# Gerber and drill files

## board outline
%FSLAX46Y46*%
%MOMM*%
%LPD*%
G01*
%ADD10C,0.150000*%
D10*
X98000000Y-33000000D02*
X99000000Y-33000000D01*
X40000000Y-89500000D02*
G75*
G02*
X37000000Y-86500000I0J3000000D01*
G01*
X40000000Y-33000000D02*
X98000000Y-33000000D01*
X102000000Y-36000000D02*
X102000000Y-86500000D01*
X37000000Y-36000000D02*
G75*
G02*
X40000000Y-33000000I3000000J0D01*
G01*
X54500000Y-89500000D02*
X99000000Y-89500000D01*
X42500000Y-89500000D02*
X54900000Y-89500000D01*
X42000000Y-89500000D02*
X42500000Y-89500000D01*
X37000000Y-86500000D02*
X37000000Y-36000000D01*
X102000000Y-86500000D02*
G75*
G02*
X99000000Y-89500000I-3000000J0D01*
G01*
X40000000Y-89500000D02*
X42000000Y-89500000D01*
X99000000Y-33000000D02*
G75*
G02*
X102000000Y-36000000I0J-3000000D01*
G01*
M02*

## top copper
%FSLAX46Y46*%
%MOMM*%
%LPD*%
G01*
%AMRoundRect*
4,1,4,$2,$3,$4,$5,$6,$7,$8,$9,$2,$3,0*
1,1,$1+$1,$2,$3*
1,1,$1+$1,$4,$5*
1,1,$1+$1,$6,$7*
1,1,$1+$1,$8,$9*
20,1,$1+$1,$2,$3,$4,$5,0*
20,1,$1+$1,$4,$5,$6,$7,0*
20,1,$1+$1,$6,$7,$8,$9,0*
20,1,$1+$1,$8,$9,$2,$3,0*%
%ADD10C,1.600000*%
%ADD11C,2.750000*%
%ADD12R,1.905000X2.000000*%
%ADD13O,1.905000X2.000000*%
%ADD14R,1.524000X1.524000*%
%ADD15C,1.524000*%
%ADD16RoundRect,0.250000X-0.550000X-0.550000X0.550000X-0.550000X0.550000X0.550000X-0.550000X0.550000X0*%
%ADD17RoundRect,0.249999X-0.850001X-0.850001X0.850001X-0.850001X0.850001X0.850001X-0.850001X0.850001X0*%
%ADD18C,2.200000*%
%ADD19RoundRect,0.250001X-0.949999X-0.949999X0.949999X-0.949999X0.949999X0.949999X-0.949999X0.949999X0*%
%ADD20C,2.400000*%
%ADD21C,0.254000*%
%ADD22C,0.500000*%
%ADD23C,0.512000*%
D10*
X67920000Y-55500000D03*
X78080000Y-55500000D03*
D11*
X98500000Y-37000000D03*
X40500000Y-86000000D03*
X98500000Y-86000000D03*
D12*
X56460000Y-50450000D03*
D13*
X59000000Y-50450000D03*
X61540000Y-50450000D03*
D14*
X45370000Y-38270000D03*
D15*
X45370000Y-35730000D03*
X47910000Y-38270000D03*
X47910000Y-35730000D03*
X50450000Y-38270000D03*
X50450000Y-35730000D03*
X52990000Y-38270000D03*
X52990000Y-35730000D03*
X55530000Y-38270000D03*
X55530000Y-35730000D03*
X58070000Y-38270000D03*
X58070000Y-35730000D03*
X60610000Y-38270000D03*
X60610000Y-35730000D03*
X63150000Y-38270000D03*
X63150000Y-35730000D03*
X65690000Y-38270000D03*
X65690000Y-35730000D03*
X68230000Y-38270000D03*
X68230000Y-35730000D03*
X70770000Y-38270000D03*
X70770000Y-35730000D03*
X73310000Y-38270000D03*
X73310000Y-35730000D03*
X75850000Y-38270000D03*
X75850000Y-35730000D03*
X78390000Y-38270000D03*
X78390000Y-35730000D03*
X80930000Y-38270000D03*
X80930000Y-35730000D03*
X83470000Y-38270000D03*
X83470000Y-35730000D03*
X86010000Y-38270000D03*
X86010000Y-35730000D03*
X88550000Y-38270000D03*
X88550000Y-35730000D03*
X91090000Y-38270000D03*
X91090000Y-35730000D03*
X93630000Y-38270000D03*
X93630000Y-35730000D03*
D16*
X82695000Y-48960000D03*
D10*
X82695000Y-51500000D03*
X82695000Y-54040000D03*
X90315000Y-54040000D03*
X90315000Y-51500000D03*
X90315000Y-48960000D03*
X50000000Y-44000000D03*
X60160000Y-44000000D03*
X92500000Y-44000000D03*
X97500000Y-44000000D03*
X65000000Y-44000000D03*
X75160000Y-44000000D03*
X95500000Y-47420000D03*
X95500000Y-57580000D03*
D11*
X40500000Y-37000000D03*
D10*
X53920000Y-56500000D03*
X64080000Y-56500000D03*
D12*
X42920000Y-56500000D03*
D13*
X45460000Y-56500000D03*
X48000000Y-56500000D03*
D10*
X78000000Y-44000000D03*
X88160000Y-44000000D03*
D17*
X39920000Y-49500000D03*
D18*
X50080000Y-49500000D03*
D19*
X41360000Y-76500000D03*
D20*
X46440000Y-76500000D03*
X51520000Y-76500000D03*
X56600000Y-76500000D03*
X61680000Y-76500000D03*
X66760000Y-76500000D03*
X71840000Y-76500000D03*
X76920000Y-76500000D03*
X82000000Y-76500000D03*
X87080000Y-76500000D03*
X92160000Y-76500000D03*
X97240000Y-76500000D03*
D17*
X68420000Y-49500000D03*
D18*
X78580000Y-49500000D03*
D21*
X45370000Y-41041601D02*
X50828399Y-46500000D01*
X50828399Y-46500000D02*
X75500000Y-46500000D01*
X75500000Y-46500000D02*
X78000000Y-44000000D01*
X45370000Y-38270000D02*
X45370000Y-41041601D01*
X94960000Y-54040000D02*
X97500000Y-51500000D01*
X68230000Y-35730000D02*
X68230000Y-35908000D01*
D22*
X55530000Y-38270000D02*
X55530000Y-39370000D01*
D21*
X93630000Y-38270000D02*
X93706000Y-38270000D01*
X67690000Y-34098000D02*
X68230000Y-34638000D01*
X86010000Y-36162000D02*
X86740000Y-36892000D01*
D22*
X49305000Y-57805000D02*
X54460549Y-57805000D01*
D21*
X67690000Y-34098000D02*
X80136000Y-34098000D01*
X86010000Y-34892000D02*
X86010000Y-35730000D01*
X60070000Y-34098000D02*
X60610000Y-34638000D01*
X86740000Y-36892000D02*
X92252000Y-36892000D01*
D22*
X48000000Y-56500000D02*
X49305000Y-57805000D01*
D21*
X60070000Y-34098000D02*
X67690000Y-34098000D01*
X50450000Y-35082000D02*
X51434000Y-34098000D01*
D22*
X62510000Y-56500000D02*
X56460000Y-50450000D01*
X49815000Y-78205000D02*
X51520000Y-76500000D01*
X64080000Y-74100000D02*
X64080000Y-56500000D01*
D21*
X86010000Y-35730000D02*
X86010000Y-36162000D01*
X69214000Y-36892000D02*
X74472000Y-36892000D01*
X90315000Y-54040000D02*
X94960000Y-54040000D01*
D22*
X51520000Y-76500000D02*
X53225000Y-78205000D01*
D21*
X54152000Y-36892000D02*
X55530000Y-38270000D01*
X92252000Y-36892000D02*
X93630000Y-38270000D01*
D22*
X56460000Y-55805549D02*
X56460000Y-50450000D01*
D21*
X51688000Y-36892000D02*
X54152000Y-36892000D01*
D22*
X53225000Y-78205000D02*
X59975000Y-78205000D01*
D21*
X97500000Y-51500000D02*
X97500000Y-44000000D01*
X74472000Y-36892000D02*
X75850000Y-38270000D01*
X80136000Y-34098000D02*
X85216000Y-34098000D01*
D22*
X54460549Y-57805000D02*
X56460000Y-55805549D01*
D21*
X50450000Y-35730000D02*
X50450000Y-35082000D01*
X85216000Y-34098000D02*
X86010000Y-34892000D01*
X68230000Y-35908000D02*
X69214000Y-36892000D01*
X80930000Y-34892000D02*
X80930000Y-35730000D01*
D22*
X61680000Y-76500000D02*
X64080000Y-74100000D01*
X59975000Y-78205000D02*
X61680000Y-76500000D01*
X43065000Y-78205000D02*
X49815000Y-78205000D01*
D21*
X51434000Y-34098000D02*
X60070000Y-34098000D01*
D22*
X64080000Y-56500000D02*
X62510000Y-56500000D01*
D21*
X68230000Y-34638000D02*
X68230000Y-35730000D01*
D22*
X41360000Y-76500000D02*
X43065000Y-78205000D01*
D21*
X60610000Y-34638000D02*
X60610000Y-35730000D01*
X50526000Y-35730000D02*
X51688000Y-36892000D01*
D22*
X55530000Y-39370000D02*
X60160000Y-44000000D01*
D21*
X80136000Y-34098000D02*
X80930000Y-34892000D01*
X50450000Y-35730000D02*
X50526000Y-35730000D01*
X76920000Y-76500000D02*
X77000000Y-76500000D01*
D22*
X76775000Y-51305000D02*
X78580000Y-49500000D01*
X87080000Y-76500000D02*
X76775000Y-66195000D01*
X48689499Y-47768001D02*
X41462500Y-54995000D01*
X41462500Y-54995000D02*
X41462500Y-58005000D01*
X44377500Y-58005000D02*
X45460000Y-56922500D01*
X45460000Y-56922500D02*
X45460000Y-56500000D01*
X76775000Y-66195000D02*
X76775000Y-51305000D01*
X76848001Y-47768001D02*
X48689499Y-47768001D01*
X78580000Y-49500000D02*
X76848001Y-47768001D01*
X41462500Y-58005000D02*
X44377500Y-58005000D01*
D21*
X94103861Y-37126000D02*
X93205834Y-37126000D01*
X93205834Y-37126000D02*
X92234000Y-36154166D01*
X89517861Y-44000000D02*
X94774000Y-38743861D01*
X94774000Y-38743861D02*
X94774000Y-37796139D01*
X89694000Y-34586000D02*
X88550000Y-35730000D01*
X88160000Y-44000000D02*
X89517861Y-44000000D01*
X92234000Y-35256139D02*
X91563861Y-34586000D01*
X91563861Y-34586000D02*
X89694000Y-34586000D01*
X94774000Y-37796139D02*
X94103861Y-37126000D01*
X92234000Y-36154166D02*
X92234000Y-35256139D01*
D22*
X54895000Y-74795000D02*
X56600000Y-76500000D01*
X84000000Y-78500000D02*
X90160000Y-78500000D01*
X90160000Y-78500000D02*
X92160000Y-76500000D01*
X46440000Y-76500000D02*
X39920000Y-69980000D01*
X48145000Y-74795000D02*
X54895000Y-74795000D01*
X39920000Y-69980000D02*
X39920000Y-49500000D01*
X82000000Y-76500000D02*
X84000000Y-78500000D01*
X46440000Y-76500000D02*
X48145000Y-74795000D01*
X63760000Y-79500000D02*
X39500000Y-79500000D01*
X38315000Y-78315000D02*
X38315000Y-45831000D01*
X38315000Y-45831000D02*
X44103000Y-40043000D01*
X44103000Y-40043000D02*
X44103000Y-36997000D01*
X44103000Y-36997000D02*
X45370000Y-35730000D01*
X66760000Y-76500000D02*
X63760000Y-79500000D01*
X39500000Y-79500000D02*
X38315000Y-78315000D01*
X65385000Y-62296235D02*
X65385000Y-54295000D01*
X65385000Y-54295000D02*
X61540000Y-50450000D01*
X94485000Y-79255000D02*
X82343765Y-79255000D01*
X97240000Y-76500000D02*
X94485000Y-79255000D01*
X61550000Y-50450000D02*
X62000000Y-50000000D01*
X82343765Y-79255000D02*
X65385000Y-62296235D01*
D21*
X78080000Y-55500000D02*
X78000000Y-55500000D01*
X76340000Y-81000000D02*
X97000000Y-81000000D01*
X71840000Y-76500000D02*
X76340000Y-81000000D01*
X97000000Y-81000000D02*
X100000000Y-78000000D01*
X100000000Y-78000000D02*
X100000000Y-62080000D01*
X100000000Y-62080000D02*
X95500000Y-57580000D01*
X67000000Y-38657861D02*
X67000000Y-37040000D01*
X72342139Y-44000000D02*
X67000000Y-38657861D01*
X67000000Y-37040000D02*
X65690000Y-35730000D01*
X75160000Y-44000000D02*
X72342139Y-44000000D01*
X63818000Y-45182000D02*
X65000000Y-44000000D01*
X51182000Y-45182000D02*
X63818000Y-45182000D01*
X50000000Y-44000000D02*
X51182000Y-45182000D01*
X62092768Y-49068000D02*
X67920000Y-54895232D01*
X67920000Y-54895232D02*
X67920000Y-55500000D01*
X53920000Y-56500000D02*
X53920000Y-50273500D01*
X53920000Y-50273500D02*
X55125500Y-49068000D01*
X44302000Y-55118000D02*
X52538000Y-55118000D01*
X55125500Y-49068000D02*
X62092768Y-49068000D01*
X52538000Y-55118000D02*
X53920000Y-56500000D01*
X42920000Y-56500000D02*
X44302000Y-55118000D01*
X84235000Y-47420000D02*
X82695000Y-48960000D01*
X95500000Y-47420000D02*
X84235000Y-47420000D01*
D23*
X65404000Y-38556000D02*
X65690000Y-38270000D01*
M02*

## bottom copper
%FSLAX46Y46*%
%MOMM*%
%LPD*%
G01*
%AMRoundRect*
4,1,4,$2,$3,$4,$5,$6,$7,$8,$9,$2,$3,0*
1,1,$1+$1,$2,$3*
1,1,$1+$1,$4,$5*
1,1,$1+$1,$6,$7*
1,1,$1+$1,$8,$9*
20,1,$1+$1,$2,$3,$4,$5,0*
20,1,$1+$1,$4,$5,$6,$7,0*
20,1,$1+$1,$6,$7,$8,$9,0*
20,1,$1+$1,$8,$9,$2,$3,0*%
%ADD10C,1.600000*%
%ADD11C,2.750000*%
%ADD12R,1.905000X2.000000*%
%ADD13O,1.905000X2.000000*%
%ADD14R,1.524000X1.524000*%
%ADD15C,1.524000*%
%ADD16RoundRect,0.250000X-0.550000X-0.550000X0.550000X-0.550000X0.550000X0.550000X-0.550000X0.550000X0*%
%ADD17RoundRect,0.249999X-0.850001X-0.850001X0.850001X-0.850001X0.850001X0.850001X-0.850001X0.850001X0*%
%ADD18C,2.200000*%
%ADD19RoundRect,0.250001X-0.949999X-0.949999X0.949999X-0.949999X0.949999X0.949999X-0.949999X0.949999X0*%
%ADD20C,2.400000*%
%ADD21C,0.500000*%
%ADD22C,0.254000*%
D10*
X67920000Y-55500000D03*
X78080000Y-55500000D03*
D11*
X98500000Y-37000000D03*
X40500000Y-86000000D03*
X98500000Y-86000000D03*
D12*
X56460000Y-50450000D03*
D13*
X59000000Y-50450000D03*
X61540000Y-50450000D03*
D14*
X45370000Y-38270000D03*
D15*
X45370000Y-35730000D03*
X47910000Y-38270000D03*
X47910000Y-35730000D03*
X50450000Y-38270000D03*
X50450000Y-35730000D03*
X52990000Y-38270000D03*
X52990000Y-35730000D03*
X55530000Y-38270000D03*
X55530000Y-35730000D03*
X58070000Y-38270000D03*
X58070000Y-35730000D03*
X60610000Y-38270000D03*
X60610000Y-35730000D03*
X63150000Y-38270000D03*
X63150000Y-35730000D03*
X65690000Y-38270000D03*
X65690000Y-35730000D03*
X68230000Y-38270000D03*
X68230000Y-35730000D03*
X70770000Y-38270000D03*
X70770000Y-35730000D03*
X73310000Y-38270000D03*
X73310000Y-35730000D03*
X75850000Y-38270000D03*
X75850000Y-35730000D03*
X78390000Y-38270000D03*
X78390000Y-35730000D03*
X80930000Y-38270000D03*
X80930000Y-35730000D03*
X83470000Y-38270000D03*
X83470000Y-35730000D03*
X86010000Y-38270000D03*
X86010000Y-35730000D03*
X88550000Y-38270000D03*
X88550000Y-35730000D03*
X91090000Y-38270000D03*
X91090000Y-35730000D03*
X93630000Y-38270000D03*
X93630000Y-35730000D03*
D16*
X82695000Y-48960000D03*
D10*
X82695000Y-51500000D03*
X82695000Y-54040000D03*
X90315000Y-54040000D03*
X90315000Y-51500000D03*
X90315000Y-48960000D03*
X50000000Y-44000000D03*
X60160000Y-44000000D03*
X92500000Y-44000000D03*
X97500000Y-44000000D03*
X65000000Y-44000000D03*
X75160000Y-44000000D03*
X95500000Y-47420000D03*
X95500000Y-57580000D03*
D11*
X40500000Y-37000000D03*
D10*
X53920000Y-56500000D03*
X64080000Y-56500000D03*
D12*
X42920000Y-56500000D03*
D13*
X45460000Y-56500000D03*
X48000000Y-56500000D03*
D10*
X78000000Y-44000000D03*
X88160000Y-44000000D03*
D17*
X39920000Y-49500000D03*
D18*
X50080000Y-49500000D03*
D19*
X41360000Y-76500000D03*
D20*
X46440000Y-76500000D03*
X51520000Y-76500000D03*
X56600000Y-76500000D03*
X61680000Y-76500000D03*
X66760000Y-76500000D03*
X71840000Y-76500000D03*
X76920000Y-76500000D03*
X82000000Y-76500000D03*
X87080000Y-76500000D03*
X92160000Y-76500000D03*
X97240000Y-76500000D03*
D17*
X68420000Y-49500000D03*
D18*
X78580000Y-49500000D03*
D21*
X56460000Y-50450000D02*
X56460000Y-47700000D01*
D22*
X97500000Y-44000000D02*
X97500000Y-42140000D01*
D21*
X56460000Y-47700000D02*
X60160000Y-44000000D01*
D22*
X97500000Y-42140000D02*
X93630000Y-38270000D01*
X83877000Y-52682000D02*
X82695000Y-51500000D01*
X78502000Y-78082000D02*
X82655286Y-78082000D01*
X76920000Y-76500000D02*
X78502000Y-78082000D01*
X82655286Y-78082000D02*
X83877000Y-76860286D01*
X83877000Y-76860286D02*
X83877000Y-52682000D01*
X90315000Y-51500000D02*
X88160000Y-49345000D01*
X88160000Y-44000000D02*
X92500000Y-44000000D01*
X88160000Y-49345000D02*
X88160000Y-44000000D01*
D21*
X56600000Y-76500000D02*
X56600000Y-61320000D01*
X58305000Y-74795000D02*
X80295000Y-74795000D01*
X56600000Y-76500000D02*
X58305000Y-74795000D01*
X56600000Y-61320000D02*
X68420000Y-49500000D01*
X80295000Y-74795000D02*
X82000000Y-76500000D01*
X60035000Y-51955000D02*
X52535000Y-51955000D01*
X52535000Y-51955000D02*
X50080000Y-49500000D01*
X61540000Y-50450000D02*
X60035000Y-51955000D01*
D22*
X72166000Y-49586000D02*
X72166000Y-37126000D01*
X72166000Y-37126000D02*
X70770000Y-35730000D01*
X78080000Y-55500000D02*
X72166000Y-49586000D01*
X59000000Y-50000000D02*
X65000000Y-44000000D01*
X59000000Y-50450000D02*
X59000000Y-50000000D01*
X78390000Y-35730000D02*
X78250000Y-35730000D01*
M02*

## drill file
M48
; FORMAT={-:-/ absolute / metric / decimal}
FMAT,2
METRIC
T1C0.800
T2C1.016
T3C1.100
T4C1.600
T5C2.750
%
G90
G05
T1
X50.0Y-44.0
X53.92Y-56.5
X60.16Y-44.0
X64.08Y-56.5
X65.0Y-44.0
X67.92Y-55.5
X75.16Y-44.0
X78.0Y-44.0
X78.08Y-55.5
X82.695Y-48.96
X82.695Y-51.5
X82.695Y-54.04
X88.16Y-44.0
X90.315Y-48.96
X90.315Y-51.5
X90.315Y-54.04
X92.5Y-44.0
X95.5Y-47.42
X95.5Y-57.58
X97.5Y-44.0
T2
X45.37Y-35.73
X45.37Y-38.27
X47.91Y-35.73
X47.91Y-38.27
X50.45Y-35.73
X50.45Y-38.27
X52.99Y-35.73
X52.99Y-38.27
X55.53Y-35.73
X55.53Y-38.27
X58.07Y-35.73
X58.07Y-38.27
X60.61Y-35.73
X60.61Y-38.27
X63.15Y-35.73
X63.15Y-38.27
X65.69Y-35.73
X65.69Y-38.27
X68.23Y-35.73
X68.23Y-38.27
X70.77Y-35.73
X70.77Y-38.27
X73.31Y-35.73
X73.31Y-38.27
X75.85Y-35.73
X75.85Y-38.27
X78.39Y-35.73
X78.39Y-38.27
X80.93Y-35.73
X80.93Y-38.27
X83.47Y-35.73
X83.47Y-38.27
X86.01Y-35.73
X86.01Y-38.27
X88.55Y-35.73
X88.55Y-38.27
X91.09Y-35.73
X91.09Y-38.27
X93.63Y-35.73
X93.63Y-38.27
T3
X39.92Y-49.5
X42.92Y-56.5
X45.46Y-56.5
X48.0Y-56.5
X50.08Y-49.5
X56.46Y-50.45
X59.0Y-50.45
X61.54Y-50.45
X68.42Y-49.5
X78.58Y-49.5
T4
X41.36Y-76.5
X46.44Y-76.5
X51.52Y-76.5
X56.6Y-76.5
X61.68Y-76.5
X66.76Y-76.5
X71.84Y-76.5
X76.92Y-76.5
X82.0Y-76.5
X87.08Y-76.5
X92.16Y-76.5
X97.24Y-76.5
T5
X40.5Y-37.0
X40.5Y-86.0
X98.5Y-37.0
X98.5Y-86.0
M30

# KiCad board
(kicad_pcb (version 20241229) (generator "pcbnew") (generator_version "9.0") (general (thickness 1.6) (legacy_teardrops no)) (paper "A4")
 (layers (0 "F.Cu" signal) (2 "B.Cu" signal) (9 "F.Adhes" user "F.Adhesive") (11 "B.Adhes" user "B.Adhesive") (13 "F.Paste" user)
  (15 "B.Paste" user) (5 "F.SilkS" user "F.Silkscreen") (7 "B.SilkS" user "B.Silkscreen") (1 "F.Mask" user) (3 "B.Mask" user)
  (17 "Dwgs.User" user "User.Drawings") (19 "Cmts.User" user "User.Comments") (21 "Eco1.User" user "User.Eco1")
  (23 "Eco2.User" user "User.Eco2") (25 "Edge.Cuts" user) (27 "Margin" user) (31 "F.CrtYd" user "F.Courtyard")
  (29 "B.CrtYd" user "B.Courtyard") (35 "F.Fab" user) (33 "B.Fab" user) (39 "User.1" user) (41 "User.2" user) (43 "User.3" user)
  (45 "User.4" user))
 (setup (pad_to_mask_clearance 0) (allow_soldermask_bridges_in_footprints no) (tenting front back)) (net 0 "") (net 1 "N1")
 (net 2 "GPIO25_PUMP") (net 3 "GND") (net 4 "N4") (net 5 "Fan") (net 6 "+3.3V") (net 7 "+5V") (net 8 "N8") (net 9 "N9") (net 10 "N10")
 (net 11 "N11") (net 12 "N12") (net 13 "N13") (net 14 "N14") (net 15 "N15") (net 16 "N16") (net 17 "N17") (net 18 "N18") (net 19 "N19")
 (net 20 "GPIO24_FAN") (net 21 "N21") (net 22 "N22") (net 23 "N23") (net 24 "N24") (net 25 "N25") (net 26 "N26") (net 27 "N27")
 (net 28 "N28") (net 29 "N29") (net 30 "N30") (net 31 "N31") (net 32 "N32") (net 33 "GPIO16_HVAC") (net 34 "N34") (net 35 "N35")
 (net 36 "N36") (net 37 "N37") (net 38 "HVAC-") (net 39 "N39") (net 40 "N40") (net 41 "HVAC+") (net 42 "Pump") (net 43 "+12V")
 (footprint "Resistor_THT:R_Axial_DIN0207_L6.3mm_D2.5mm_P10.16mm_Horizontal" (layer "F.Cu") (at 67.92 55.5)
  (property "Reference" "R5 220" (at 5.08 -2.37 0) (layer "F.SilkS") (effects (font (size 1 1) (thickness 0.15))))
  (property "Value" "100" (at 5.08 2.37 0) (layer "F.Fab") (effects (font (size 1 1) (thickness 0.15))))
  (pad "1" thru_hole circle (at 0 0) (size 1.6 1.6) (drill 0.8) (layers "*.Cu" "*.Mask") (remove_unused_layers no) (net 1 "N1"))
  (pad "2" thru_hole circle (at 10.16 0) (size 1.6 1.6) (drill 0.8) (layers "*.Cu" "*.Mask") (remove_unused_layers no) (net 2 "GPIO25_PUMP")))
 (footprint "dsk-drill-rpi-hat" (layer "F.Cu") (at 98.5 37)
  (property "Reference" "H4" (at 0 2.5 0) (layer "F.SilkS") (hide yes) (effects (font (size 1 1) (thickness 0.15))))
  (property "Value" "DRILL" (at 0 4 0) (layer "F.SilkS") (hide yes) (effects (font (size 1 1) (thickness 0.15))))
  (pad "1" thru_hole circle (at 0 0) (size 2.75 2.75) (drill 2.75) (layers "*.Cu") (remove_unused_layers no) (solder_mask_margin 1.725)
   (clearance 1.725) (zone_connect 0)))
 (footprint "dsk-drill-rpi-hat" (layer "F.Cu") (at 40.5 86)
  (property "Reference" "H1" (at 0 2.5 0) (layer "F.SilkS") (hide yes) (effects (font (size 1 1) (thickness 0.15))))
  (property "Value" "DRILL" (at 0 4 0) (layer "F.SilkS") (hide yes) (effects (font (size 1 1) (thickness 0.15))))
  (pad "1" thru_hole circle (at 0 0) (size 2.75 2.75) (drill 2.75) (layers "*.Cu") (remove_unused_layers no) (solder_mask_margin 1.725)
   (clearance 1.725) (zone_connect 0)))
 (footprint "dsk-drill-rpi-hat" (layer "F.Cu") (at 98.5 86)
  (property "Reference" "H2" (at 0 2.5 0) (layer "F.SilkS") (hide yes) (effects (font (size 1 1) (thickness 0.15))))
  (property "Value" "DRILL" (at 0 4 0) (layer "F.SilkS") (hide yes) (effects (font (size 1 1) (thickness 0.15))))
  (pad "1" thru_hole circle (at 0 0) (size 2.75 2.75) (drill 2.75) (layers "*.Cu") (remove_unused_layers no) (solder_mask_margin 1.725)
   (clearance 1.725) (zone_connect 0)))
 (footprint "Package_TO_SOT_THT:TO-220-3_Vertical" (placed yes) (layer "F.Cu") (at 56.46 50.45)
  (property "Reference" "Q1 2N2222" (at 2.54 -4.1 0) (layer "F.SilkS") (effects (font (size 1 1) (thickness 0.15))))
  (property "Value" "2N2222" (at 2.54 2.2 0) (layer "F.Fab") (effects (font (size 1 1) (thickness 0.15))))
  (pad "1" thru_hole rect (at 0 0) (size 1.905 2) (drill 1.1) (layers "*.Cu" "*.Mask") (remove_unused_layers no) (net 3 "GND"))
  (pad "2" thru_hole oval (at 2.54 0) (size 1.905 2) (drill 1.1) (layers "*.Cu" "*.Mask") (remove_unused_layers no) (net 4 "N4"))
  (pad "3" thru_hole oval (at 5.08 0) (size 1.905 2) (drill 1.1) (layers "*.Cu" "*.Mask") (remove_unused_layers no) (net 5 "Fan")))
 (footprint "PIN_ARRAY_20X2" (layer "F.Cu") (at 69.5 37)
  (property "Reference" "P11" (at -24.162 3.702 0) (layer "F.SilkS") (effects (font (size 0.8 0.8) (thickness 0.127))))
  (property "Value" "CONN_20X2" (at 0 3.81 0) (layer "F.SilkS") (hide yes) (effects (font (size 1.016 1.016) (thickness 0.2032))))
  (pad "1" thru_hole rect (at -24.13 1.27) (size 1.524 1.524) (drill 1.016) (layers "*.Cu" "*.Mask" "F.SilkS") (remove_unused_layers no)
   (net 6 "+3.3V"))
  (pad "2" thru_hole circle (at -24.13 -1.27) (size 1.524 1.524) (drill 1.016) (layers "*.Cu" "*.Mask" "F.SilkS") (remove_unused_layers no)
   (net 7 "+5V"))
  (pad "3" thru_hole circle (at -21.59 1.27) (size 1.524 1.524) (drill 1.016) (layers "*.Cu" "*.Mask" "F.SilkS") (remove_unused_layers no)
   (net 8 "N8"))
  (pad "4" thru_hole circle (at -21.59 -1.27) (size 1.524 1.524) (drill 1.016) (layers "*.Cu" "*.Mask" "F.SilkS") (remove_unused_layers no)
   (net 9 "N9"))
  (pad "5" thru_hole circle (at -19.05 1.27) (size 1.524 1.524) (drill 1.016) (layers "*.Cu" "*.Mask" "F.SilkS") (remove_unused_layers no)
   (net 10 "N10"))
  (pad "6" thru_hole circle (at -19.05 -1.27) (size 1.524 1.524) (drill 1.016) (layers "*.Cu" "*.Mask" "F.SilkS") (remove_unused_layers no)
   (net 3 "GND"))
  (pad "7" thru_hole circle (at -16.51 1.27) (size 1.524 1.524) (drill 1.016) (layers "*.Cu" "*.Mask" "F.SilkS") (remove_unused_layers no)
   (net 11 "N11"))
  (pad "8" thru_hole circle (at -16.51 -1.27) (size 1.524 1.524) (drill 1.016) (layers "*.Cu" "*.Mask" "F.SilkS") (remove_unused_layers no)
   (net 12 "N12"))
  (pad "9" thru_hole circle (at -13.97 1.27) (size 1.524 1.524) (drill 1.016) (layers "*.Cu" "*.Mask" "F.SilkS") (remove_unused_layers no)
   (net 3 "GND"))
  (pad "10" thru_hole circle (at -13.97 -1.27) (size 1.524 1.524) (drill 1.016) (layers "*.Cu" "*.Mask" "F.SilkS") (remove_unused_layers no)
   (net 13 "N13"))
  (pad "11" thru_hole circle (at -11.43 1.27) (size 1.524 1.524) (drill 1.016) (layers "*.Cu" "*.Mask" "F.SilkS") (remove_unused_layers no)
   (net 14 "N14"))
  (pad "12" thru_hole circle (at -11.43 -1.27) (size 1.524 1.524) (drill 1.016) (layers "*.Cu" "*.Mask" "F.SilkS") (remove_unused_layers no)
   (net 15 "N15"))
  (pad "13" thru_hole circle (at -8.89 1.27) (size 1.524 1.524) (drill 1.016) (layers "*.Cu" "*.Mask" "F.SilkS") (remove_unused_layers no)
   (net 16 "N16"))
  (pad "14" thru_hole circle (at -8.89 -1.27) (size 1.524 1.524) (drill 1.016) (layers "*.Cu" "*.Mask" "F.SilkS") (remove_unused_layers no)
   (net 3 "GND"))
  (pad "15" thru_hole circle (at -6.35 1.27) (size 1.524 1.524) (drill 1.016) (layers "*.Cu" "*.Mask" "F.SilkS") (remove_unused_layers no)
   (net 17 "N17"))
  (pad "16" thru_hole circle (at -6.35 -1.27) (size 1.524 1.524) (drill 1.016) (layers "*.Cu" "*.Mask" "F.SilkS") (remove_unused_layers no)
   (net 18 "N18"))
  (pad "17" thru_hole circle (at -3.81 1.27) (size 1.524 1.524) (drill 1.016) (layers "*.Cu" "*.Mask" "F.SilkS") (remove_unused_layers no)
   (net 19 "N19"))
  (pad "18" thru_hole circle (at -3.81 -1.27) (size 1.524 1.524) (drill 1.016) (layers "*.Cu" "*.Mask" "F.SilkS") (remove_unused_layers no)
   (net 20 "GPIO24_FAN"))
  (pad "19" thru_hole circle (at -1.27 1.27) (size 1.524 1.524) (drill 1.016) (layers "*.Cu" "*.Mask" "F.SilkS") (remove_unused_layers no)
   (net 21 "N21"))
  (pad "20" thru_hole circle (at -1.27 -1.27) (size 1.524 1.524) (drill 1.016) (layers "*.Cu" "*.Mask" "F.SilkS") (remove_unused_layers no)
   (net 3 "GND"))
  (pad "21" thru_hole circle (at 1.27 1.27) (size 1.524 1.524) (drill 1.016) (layers "*.Cu" "*.Mask" "F.SilkS") (remove_unused_layers no)
   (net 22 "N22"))
  (pad "22" thru_hole circle (at 1.27 -1.27) (size 1.524 1.524) (drill 1.016) (layers "*.Cu" "*.Mask" "F.SilkS") (remove_unused_layers no)
   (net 2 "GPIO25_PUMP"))
  (pad "23" thru_hole circle (at 3.81 1.27) (size 1.524 1.524) (drill 1.016) (layers "*.Cu" "*.Mask" "F.SilkS") (remove_unused_layers no)
   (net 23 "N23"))
  (pad "24" thru_hole circle (at 3.81 -1.27) (size 1.524 1.524) (drill 1.016) (layers "*.Cu" "*.Mask" "F.SilkS") (remove_unused_layers no)
   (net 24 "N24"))
  (pad "25" thru_hole circle (at 6.35 1.27) (size 1.524 1.524) (drill 1.016) (layers "*.Cu" "*.Mask" "F.SilkS") (remove_unused_layers no)
   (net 3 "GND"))
  (pad "26" thru_hole circle (at 6.35 -1.27) (size 1.524 1.524) (drill 1.016) (layers "*.Cu" "*.Mask" "F.SilkS") (remove_unused_layers no)
   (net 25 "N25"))
  (pad "27" thru_hole circle (at 8.89 1.27) (size 1.524 1.524) (drill 1.016) (layers "*.Cu" "*.Mask" "F.SilkS") (remove_unused_layers no)
   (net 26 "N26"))
  (pad "28" thru_hole circle (at 8.89 -1.27) (size 1.524 1.524) (drill 1.016) (layers "*.Cu" "*.Mask" "F.SilkS") (remove_unused_layers no)
   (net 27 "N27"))
  (pad "29" thru_hole circle (at 11.43 1.27) (size 1.524 1.524) (drill 1.016) (layers "*.Cu" "*.Mask" "F.SilkS") (remove_unused_layers no)
   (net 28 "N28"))
  (pad "30" thru_hole circle (at 11.43 -1.27) (size 1.524 1.524) (drill 1.016) (layers "*.Cu" "*.Mask" "F.SilkS") (remove_unused_layers no)
   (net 3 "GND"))
  (pad "31" thru_hole circle (at 13.97 1.27) (size 1.524 1.524) (drill 1.016) (layers "*.Cu" "*.Mask" "F.SilkS") (remove_unused_layers no)
   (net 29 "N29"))
  (pad "32" thru_hole circle (at 13.97 -1.27) (size 1.524 1.524) (drill 1.016) (layers "*.Cu" "*.Mask" "F.SilkS") (remove_unused_layers no)
   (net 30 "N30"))
  (pad "33" thru_hole circle (at 16.51 1.27) (size 1.524 1.524) (drill 1.016) (layers "*.Cu" "*.Mask" "F.SilkS") (remove_unused_layers no)
   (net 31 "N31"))
  (pad "34" thru_hole circle (at 16.51 -1.27) (size 1.524 1.524) (drill 1.016) (layers "*.Cu" "*.Mask" "F.SilkS") (remove_unused_layers no)
   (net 3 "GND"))
  (pad "35" thru_hole circle (at 19.05 1.27) (size 1.524 1.524) (drill 1.016) (layers "*.Cu" "*.Mask" "F.SilkS") (remove_unused_layers no)
   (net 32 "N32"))
  (pad "36" thru_hole circle (at 19.05 -1.27) (size 1.524 1.524) (drill 1.016) (layers "*.Cu" "*.Mask" "F.SilkS") (remove_unused_layers no)
   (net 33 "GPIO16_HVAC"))
  (pad "37" thru_hole circle (at 21.59 1.27) (size 1.524 1.524) (drill 1.016) (layers "*.Cu" "*.Mask" "F.SilkS") (remove_unused_layers no)
   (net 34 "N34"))
  (pad "38" thru_hole circle (at 21.59 -1.27) (size 1.524 1.524) (drill 1.016) (layers "*.Cu" "*.Mask" "F.SilkS") (remove_unused_layers no)
   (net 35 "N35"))
  (pad "39" thru_hole circle (at 24.13 1.27) (size 1.524 1.524) (drill 1.016) (layers "*.Cu" "*.Mask" "F.SilkS") (remove_unused_layers no)
   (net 3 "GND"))
  (pad "40" thru_hole circle (at 24.13 -1.27) (size 1.524 1.524) (drill 1.016) (layers "*.Cu" "*.Mask" "F.SilkS") (remove_unused_layers no)
   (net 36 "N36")))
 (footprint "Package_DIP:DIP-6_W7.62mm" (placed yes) (layer "F.Cu") (at 82.695 48.96)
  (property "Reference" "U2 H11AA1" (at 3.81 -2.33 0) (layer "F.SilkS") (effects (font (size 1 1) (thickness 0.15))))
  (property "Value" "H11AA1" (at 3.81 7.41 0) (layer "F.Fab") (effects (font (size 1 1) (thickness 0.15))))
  (pad "1" thru_hole roundrect (at 0 0) (size 1.6 1.6) (drill 0.8) (layers "*.Cu" "*.Mask") (remove_unused_layers no)
   (roundrect_rratio 0.15625) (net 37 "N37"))
  (pad "2" thru_hole circle (at 0 2.54) (size 1.6 1.6) (drill 0.8) (layers "*.Cu" "*.Mask") (remove_unused_layers no) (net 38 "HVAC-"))
  (pad "3" thru_hole circle (at 0 5.08) (size 1.6 1.6) (drill 0.8) (layers "*.Cu" "*.Mask") (remove_unused_layers no) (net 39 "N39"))
  (pad "4" thru_hole circle (at 7.62 5.08) (size 1.6 1.6) (drill 0.8) (layers "*.Cu" "*.Mask") (remove_unused_layers no) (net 3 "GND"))
  (pad "5" thru_hole circle (at 7.62 2.54) (size 1.6 1.6) (drill 0.8) (layers "*.Cu" "*.Mask") (remove_unused_layers no)
   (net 33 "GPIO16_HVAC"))
  (pad "6" thru_hole circle (at 7.62 0) (size 1.6 1.6) (drill 0.8) (layers "*.Cu" "*.Mask") (remove_unused_layers no) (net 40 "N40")))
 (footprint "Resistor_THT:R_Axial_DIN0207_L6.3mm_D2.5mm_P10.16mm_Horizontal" (layer "F.Cu") (at 50 44)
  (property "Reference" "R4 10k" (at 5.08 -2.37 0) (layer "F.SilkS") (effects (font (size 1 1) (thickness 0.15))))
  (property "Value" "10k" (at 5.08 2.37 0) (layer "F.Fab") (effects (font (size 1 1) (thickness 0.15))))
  (pad "1" thru_hole circle (at 0 0) (size 1.6 1.6) (drill 0.8) (layers "*.Cu" "*.Mask") (remove_unused_layers no) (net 4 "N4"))
  (pad "2" thru_hole circle (at 10.16 0) (size 1.6 1.6) (drill 0.8) (layers "*.Cu" "*.Mask") (remove_unused_layers no) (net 3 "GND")))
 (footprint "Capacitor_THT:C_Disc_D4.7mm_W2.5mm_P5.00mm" (layer "F.Cu") (at 92.5 44)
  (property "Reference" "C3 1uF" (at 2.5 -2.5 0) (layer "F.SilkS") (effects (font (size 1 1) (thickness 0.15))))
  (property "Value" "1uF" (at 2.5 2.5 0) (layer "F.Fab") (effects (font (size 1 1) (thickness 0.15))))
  (pad "1" thru_hole circle (at 0 0) (size 1.6 1.6) (drill 0.8) (layers "*.Cu" "*.Mask") (remove_unused_layers no) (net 33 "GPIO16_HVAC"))
  (pad "2" thru_hole circle (at 5 0) (size 1.6 1.6) (drill 0.8) (layers "*.Cu" "*.Mask") (remove_unused_layers no) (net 3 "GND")))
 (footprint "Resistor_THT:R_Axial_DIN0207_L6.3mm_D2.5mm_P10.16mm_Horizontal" (layer "F.Cu") (at 65 44)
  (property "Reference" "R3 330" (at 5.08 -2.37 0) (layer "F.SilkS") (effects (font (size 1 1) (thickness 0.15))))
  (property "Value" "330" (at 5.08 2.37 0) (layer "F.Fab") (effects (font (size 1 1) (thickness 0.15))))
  (pad "1" thru_hole circle (at 0 0) (size 1.6 1.6) (drill 0.8) (layers "*.Cu" "*.Mask") (remove_unused_layers no) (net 4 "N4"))
  (pad "2" thru_hole circle (at 10.16 0) (size 1.6 1.6) (drill 0.8) (layers "*.Cu" "*.Mask") (remove_unused_layers no) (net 20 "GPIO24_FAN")))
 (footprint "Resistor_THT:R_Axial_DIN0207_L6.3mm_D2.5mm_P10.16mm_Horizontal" (layer "F.Cu") (at 95.5 47.42 -90)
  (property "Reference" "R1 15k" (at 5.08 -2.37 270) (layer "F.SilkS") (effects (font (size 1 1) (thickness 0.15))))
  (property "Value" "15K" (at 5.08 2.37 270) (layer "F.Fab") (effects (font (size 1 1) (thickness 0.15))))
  (pad "1" thru_hole circle (at 0 0 270) (size 1.6 1.6) (drill 0.8) (layers "*.Cu" "*.Mask") (remove_unused_layers no) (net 37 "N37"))
  (pad "2" thru_hole circle (at 10.16 0 270) (size 1.6 1.6) (drill 0.8) (layers "*.Cu" "*.Mask") (remove_unused_layers no) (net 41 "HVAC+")))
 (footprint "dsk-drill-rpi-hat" (layer "F.Cu") (at 40.5 37)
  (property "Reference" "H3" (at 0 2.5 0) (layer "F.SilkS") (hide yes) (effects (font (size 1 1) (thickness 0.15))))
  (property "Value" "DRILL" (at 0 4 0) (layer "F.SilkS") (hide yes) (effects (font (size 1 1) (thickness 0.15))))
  (pad "1" thru_hole circle (at 0 0) (size 2.75 2.75) (drill 2.75) (layers "*.Cu") (remove_unused_layers no) (solder_mask_margin 1.725)
   (clearance 1.725) (zone_connect 0)))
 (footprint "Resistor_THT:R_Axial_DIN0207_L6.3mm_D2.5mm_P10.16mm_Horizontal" (layer "F.Cu") (at 53.92 56.5)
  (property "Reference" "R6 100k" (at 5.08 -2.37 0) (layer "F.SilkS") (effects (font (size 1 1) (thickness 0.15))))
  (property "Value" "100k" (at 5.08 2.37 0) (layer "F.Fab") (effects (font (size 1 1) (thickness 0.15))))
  (pad "1" thru_hole circle (at 0 0) (size 1.6 1.6) (drill 0.8) (layers "*.Cu" "*.Mask") (remove_unused_layers no) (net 1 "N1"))
  (pad "2" thru_hole circle (at 10.16 0) (size 1.6 1.6) (drill 0.8) (layers "*.Cu" "*.Mask") (remove_unused_layers no) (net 3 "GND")))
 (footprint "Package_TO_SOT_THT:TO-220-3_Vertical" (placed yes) (layer "F.Cu") (at 42.92 56.5)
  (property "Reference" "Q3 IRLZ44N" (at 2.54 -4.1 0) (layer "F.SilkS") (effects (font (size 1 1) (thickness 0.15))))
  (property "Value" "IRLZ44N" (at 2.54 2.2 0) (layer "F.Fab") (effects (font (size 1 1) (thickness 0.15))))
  (pad "1" thru_hole rect (at 0 0) (size 1.905 2) (drill 1.1) (layers "*.Cu" "*.Mask") (remove_unused_layers no) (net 1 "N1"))
  (pad "2" thru_hole oval (at 2.54 0) (size 1.905 2) (drill 1.1) (layers "*.Cu" "*.Mask") (remove_unused_layers no) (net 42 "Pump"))
  (pad "3" thru_hole oval (at 5.08 0) (size 1.905 2) (drill 1.1) (layers "*.Cu" "*.Mask") (remove_unused_layers no) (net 3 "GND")))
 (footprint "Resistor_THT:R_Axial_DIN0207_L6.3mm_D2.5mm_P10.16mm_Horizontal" (layer "F.Cu") (at 78 44)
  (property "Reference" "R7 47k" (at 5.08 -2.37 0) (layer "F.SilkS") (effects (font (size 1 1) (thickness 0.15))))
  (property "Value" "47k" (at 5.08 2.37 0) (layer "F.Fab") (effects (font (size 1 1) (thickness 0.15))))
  (pad "1" thru_hole circle (at 0 0) (size 1.6 1.6) (drill 0.8) (layers "*.Cu" "*.Mask") (remove_unused_layers no) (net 6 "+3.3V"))
  (pad "2" thru_hole circle (at 10.16 0) (size 1.6 1.6) (drill 0.8) (layers "*.Cu" "*.Mask") (remove_unused_layers no)
   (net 33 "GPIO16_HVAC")))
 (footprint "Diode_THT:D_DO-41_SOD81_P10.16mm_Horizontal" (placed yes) (layer "F.Cu") (at 39.92 49.5)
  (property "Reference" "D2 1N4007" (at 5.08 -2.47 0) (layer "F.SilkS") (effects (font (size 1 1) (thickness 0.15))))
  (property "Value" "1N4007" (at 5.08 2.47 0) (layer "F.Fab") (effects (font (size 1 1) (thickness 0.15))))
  (pad "1" thru_hole roundrect (at 0 0) (size 2.2 2.2) (drill 1.1) (layers "*.Cu" "*.Mask") (remove_unused_layers no)
   (roundrect_rratio 0.113636) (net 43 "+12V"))
  (pad "2" thru_hole circle (at 10.16 0) (size 2.2 2.2) (drill 1.1) (layers "*.Cu" "*.Mask") (remove_unused_layers no) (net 5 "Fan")))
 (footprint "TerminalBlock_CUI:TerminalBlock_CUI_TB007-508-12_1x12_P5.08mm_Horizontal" (layer "F.Cu") (at 41.36 76.5)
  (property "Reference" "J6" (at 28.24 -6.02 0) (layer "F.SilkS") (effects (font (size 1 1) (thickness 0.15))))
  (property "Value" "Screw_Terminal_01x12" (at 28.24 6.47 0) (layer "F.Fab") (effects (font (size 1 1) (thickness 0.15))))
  (pad "1" thru_hole roundrect (at 0 0) (size 2.4 2.4) (drill 1.6) (layers "*.Cu" "*.Mask") (remove_unused_layers no)
   (roundrect_rratio 0.104167) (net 3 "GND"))
  (pad "2" thru_hole circle (at 5.08 0) (size 2.4 2.4) (drill 1.6) (layers "*.Cu" "*.Mask") (remove_unused_layers no) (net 43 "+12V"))
  (pad "3" thru_hole circle (at 10.16 0) (size 2.4 2.4) (drill 1.6) (layers "*.Cu" "*.Mask") (remove_unused_layers no) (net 3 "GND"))
  (pad "4" thru_hole circle (at 15.24 0) (size 2.4 2.4) (drill 1.6) (layers "*.Cu" "*.Mask") (remove_unused_layers no) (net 43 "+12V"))
  (pad "5" thru_hole circle (at 20.32 0) (size 2.4 2.4) (drill 1.6) (layers "*.Cu" "*.Mask") (remove_unused_layers no) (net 3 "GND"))
  (pad "6" thru_hole circle (at 25.4 0) (size 2.4 2.4) (drill 1.6) (layers "*.Cu" "*.Mask") (remove_unused_layers no) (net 7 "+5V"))
  (pad "7" thru_hole circle (at 30.48 0) (size 2.4 2.4) (drill 1.6) (layers "*.Cu" "*.Mask") (remove_unused_layers no) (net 41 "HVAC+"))
  (pad "8" thru_hole circle (at 35.56 0) (size 2.4 2.4) (drill 1.6) (layers "*.Cu" "*.Mask") (remove_unused_layers no) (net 38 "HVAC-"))
  (pad "9" thru_hole circle (at 40.64 0) (size 2.4 2.4) (drill 1.6) (layers "*.Cu" "*.Mask") (remove_unused_layers no) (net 43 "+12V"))
  (pad "10" thru_hole circle (at 45.72 0) (size 2.4 2.4) (drill 1.6) (layers "*.Cu" "*.Mask") (remove_unused_layers no) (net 42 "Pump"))
  (pad "11" thru_hole circle (at 50.8 0) (size 2.4 2.4) (drill 1.6) (layers "*.Cu" "*.Mask") (remove_unused_layers no) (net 43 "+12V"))
  (pad "12" thru_hole circle (at 55.88 0) (size 2.4 2.4) (drill 1.6) (layers "*.Cu" "*.Mask") (remove_unused_layers no) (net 5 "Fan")))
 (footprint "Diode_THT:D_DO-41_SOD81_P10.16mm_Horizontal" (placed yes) (layer "F.Cu") (at 68.42 49.5)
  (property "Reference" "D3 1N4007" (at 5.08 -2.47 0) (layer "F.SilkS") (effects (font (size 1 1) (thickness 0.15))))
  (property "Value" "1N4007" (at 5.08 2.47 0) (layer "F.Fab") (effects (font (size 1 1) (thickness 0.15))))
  (pad "1" thru_hole roundrect (at 0 0) (size 2.2 2.2) (drill 1.1) (layers "*.Cu" "*.Mask") (remove_unused_layers no)
   (roundrect_rratio 0.113636) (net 43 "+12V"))
  (pad "2" thru_hole circle (at 10.16 0) (size 2.2 2.2) (drill 1.1) (layers "*.Cu" "*.Mask") (remove_unused_layers no) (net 42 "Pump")))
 (gr_line (start 98 33) (end 99 33) (stroke (width 0.15) (type solid)) (layer "Edge.Cuts"))
 (gr_arc (start 40 89.5) (mid 37.87868 88.62132) (end 37 86.5) (stroke (width 0.15) (type solid)) (layer "Edge.Cuts"))
 (gr_line (start 40 33) (end 98 33) (stroke (width 0.15) (type solid)) (layer "Edge.Cuts"))
 (gr_line (start 102 36) (end 102 86.5) (stroke (width 0.15) (type solid)) (layer "Edge.Cuts"))
 (gr_arc (start 37 36) (mid 37.87868 33.87868) (end 40 33) (stroke (width 0.15) (type solid)) (layer "Edge.Cuts"))
 (gr_line (start 54.5 89.5) (end 99 89.5) (stroke (width 0.15) (type solid)) (layer "Edge.Cuts"))
 (gr_line (start 42.5 89.5) (end 54.9 89.5) (stroke (width 0.15) (type solid)) (layer "Edge.Cuts"))
 (gr_line (start 42 89.5) (end 42.5 89.5) (stroke (width 0.15) (type solid)) (layer "Edge.Cuts"))
 (gr_line (start 37 86.5) (end 37 36) (stroke (width 0.15) (type solid)) (layer "Edge.Cuts"))
 (gr_arc (start 102 86.5) (mid 101.12132 88.62132) (end 99 89.5) (stroke (width 0.15) (type solid)) (layer "Edge.Cuts"))
 (gr_line (start 40 89.5) (end 42 89.5) (stroke (width 0.15) (type solid)) (layer "Edge.Cuts"))
 (gr_arc (start 99 33) (mid 101.12132 33.87868) (end 102 36) (stroke (width 0.15) (type solid)) (layer "Edge.Cuts"))
 (segment (start 45.37 41.041601) (end 50.828399 46.5) (width 0.254) (layer "F.Cu") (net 6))
 (segment (start 50.828399 46.5) (end 75.5 46.5) (width 0.254) (layer "F.Cu") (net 6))
 (segment (start 75.5 46.5) (end 78 44) (width 0.254) (layer "F.Cu") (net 6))
 (segment (start 45.37 38.27) (end 45.37 41.041601) (width 0.254) (layer "F.Cu") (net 6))
 (segment (start 94.96 54.04) (end 97.5 51.5) (width 0.254) (layer "F.Cu") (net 3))
 (segment (start 68.23 35.73) (end 68.23 35.908) (width 0.254) (layer "F.Cu") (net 3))
 (segment (start 55.53 38.27) (end 55.53 39.37) (width 0.5) (layer "F.Cu") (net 3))
 (segment (start 93.63 38.27) (end 93.706 38.27) (width 0.254) (layer "F.Cu") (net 3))
 (segment (start 67.69 34.098) (end 68.23 34.638) (width 0.254) (layer "F.Cu") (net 3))
 (segment (start 86.01 36.162) (end 86.74 36.892) (width 0.254) (layer "F.Cu") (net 3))
 (segment (start 49.305 57.805) (end 54.460549 57.805) (width 0.5) (layer "F.Cu") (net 3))
 (segment (start 67.69 34.098) (end 80.136 34.098) (width 0.254) (layer "F.Cu") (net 3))
 (segment (start 86.01 34.892) (end 86.01 35.73) (width 0.254) (layer "F.Cu") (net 3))
 (segment (start 60.07 34.098) (end 60.61 34.638) (width 0.254) (layer "F.Cu") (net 3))
 (segment (start 86.74 36.892) (end 92.252 36.892) (width 0.254) (layer "F.Cu") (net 3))
 (segment (start 48 56.5) (end 49.305 57.805) (width 0.5) (layer "F.Cu") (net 3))
 (segment (start 60.07 34.098) (end 67.69 34.098) (width 0.254) (layer "F.Cu") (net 3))
 (segment (start 50.45 35.082) (end 51.434 34.098) (width 0.254) (layer "F.Cu") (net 3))
 (segment (start 62.51 56.5) (end 56.46 50.45) (width 0.5) (layer "F.Cu") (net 3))
 (segment (start 49.815 78.205) (end 51.52 76.5) (width 0.5) (layer "F.Cu") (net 3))
 (segment (start 64.08 74.1) (end 64.08 56.5) (width 0.5) (layer "F.Cu") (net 3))
 (segment (start 86.01 35.73) (end 86.01 36.162) (width 0.254) (layer "F.Cu") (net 3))
 (segment (start 69.214 36.892) (end 74.472 36.892) (width 0.254) (layer "F.Cu") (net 3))
 (segment (start 90.315 54.04) (end 94.96 54.04) (width 0.254) (layer "F.Cu") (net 3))
 (segment (start 51.52 76.5) (end 53.225 78.205) (width 0.5) (layer "F.Cu") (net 3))
 (segment (start 54.152 36.892) (end 55.53 38.27) (width 0.254) (layer "F.Cu") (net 3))
 (segment (start 92.252 36.892) (end 93.63 38.27) (width 0.254) (layer "F.Cu") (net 3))
 (segment (start 56.46 55.805549) (end 56.46 50.45) (width 0.5) (layer "F.Cu") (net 3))
 (segment (start 51.688 36.892) (end 54.152 36.892) (width 0.254) (layer "F.Cu") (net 3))
 (segment (start 53.225 78.205) (end 59.975 78.205) (width 0.5) (layer "F.Cu") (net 3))
 (segment (start 97.5 51.5) (end 97.5 44) (width 0.254) (layer "F.Cu") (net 3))
 (segment (start 74.472 36.892) (end 75.85 38.27) (width 0.254) (layer "F.Cu") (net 3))
 (segment (start 80.136 34.098) (end 85.216 34.098) (width 0.254) (layer "F.Cu") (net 3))
 (segment (start 54.460549 57.805) (end 56.46 55.805549) (width 0.5) (layer "F.Cu") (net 3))
 (segment (start 50.45 35.73) (end 50.45 35.082) (width 0.254) (layer "F.Cu") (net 3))
 (segment (start 85.216 34.098) (end 86.01 34.892) (width 0.254) (layer "F.Cu") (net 3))
 (segment (start 68.23 35.908) (end 69.214 36.892) (width 0.254) (layer "F.Cu") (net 3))
 (segment (start 80.93 34.892) (end 80.93 35.73) (width 0.254) (layer "F.Cu") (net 3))
 (segment (start 61.68 76.5) (end 64.08 74.1) (width 0.5) (layer "F.Cu") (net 3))
 (segment (start 59.975 78.205) (end 61.68 76.5) (width 0.5) (layer "F.Cu") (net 3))
 (segment (start 43.065 78.205) (end 49.815 78.205) (width 0.5) (layer "F.Cu") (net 3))
 (segment (start 51.434 34.098) (end 60.07 34.098) (width 0.254) (layer "F.Cu") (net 3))
 (segment (start 64.08 56.5) (end 62.51 56.5) (width 0.5) (layer "F.Cu") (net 3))
 (segment (start 68.23 34.638) (end 68.23 35.73) (width 0.254) (layer "F.Cu") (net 3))
 (segment (start 41.36 76.5) (end 43.065 78.205) (width 0.5) (layer "F.Cu") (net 3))
 (segment (start 60.61 34.638) (end 60.61 35.73) (width 0.254) (layer "F.Cu") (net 3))
 (segment (start 50.526 35.73) (end 51.688 36.892) (width 0.254) (layer "F.Cu") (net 3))
 (segment (start 55.53 39.37) (end 60.16 44) (width 0.5) (layer "F.Cu") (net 3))
 (segment (start 80.136 34.098) (end 80.93 34.892) (width 0.254) (layer "F.Cu") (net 3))
 (segment (start 50.45 35.73) (end 50.526 35.73) (width 0.254) (layer "F.Cu") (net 3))
 (segment (start 56.46 50.45) (end 56.46 47.7) (width 0.5) (layer "B.Cu") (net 3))
 (segment (start 97.5 44) (end 97.5 42.14) (width 0.254) (layer "B.Cu") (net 3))
 (segment (start 56.46 47.7) (end 60.16 44) (width 0.5) (layer "B.Cu") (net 3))
 (segment (start 97.5 42.14) (end 93.63 38.27) (width 0.254) (layer "B.Cu") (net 3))
 (segment (start 76.92 76.5) (end 77 76.5) (width 0.254) (layer "F.Cu") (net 38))
 (segment (start 83.877 52.682) (end 82.695 51.5) (width 0.254) (layer "B.Cu") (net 38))
 (segment (start 78.502 78.082) (end 82.655286 78.082) (width 0.254) (layer "B.Cu") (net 38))
 (segment (start 76.92 76.5) (end 78.502 78.082) (width 0.254) (layer "B.Cu") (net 38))
 (segment (start 82.655286 78.082) (end 83.877 76.860286) (width 0.254) (layer "B.Cu") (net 38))
 (segment (start 83.877 76.860286) (end 83.877 52.682) (width 0.254) (layer "B.Cu") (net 38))
 (segment (start 76.775 51.305) (end 78.58 49.5) (width 0.5) (layer "F.Cu") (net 42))
 (segment (start 87.08 76.5) (end 76.775 66.195) (width 0.5) (layer "F.Cu") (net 42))
 (segment (start 48.689499 47.768001) (end 41.4625 54.995) (width 0.5) (layer "F.Cu") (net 42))
 (segment (start 41.4625 54.995) (end 41.4625 58.005) (width 0.5) (layer "F.Cu") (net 42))
 (segment (start 44.3775 58.005) (end 45.46 56.9225) (width 0.5) (layer "F.Cu") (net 42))
 (segment (start 45.46 56.9225) (end 45.46 56.5) (width 0.5) (layer "F.Cu") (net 42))
 (segment (start 76.775 66.195) (end 76.775 51.305) (width 0.5) (layer "F.Cu") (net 42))
 (segment (start 76.848001 47.768001) (end 48.689499 47.768001) (width 0.5) (layer "F.Cu") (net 42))
 (segment (start 78.58 49.5) (end 76.848001 47.768001) (width 0.5) (layer "F.Cu") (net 42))
 (segment (start 41.4625 58.005) (end 44.3775 58.005) (width 0.5) (layer "F.Cu") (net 42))
 (segment (start 94.103861 37.126) (end 93.205834 37.126) (width 0.254) (layer "F.Cu") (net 33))
 (segment (start 93.205834 37.126) (end 92.234 36.154166) (width 0.254) (layer "F.Cu") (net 33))
 (segment (start 89.517861 44) (end 94.774 38.743861) (width 0.254) (layer "F.Cu") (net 33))
 (segment (start 94.774 38.743861) (end 94.774 37.796139) (width 0.254) (layer "F.Cu") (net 33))
 (segment (start 89.694 34.586) (end 88.55 35.73) (width 0.254) (layer "F.Cu") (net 33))
 (segment (start 88.16 44) (end 89.517861 44) (width 0.254) (layer "F.Cu") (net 33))
 (segment (start 92.234 35.256139) (end 91.563861 34.586) (width 0.254) (layer "F.Cu") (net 33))
 (segment (start 91.563861 34.586) (end 89.694 34.586) (width 0.254) (layer "F.Cu") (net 33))
 (segment (start 94.774 37.796139) (end 94.103861 37.126) (width 0.254) (layer "F.Cu") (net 33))
 (segment (start 92.234 36.154166) (end 92.234 35.256139) (width 0.254) (layer "F.Cu") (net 33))
 (segment (start 90.315 51.5) (end 88.16 49.345) (width 0.254) (layer "B.Cu") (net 33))
 (segment (start 88.16 44) (end 92.5 44) (width 0.254) (layer "B.Cu") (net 33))
 (segment (start 88.16 49.345) (end 88.16 44) (width 0.254) (layer "B.Cu") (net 33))
 (segment (start 54.895 74.795) (end 56.6 76.5) (width 0.5) (layer "F.Cu") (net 43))
 (segment (start 84 78.5) (end 90.16 78.5) (width 0.5) (layer "F.Cu") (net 43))
 (segment (start 90.16 78.5) (end 92.16 76.5) (width 0.5) (layer "F.Cu") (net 43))
 (segment (start 46.44 76.5) (end 39.92 69.98) (width 0.5) (layer "F.Cu") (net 43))
 (segment (start 48.145 74.795) (end 54.895 74.795) (width 0.5) (layer "F.Cu") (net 43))
 (segment (start 39.92 69.98) (end 39.92 49.5) (width 0.5) (layer "F.Cu") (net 43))
 (segment (start 82 76.5) (end 84 78.5) (width 0.5) (layer "F.Cu") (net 43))
 (segment (start 46.44 76.5) (end 48.145 74.795) (width 0.5) (layer "F.Cu") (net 43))
 (segment (start 56.6 76.5) (end 56.6 61.32) (width 0.5) (layer "B.Cu") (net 43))
 (segment (start 58.305 74.795) (end 80.295 74.795) (width 0.5) (layer "B.Cu") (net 43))
 (segment (start 56.6 76.5) (end 58.305 74.795) (width 0.5) (layer "B.Cu") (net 43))
 (segment (start 56.6 61.32) (end 68.42 49.5) (width 0.5) (layer "B.Cu") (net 43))
 (segment (start 80.295 74.795) (end 82 76.5) (width 0.5) (layer "B.Cu") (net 43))
 (segment (start 63.76 79.5) (end 39.5 79.5) (width 0.5) (layer "F.Cu") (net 7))
 (segment (start 38.315 78.315) (end 38.315 45.831) (width 0.5) (layer "F.Cu") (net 7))
 (segment (start 38.315 45.831) (end 44.103 40.043) (width 0.5) (layer "F.Cu") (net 7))
 (segment (start 44.103 40.043) (end 44.103 36.997) (width 0.5) (layer "F.Cu") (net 7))
 (segment (start 44.103 36.997) (end 45.37 35.73) (width 0.5) (layer "F.Cu") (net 7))
 (segment (start 66.76 76.5) (end 63.76 79.5) (width 0.5) (layer "F.Cu") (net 7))
 (segment (start 39.5 79.5) (end 38.315 78.315) (width 0.5) (layer "F.Cu") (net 7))
 (segment (start 65.385 62.296235) (end 65.385 54.295) (width 0.5) (layer "F.Cu") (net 5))
 (segment (start 65.385 54.295) (end 61.54 50.45) (width 0.5) (layer "F.Cu") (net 5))
 (segment (start 94.485 79.255) (end 82.343765 79.255) (width 0.5) (layer "F.Cu") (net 5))
 (segment (start 97.24 76.5) (end 94.485 79.255) (width 0.5) (layer "F.Cu") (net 5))
 (segment (start 61.55 50.45) (end 62 50) (width 0.5) (layer "F.Cu") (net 5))
 (segment (start 82.343765 79.255) (end 65.385 62.296235) (width 0.5) (layer "F.Cu") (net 5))
 (segment (start 60.035 51.955) (end 52.535 51.955) (width 0.5) (layer "B.Cu") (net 5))
 (segment (start 52.535 51.955) (end 50.08 49.5) (width 0.5) (layer "B.Cu") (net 5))
 (segment (start 61.54 50.45) (end 60.035 51.955) (width 0.5) (layer "B.Cu") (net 5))
 (segment (start 78.08 55.5) (end 78 55.5) (width 0.254) (layer "F.Cu") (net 2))
 (segment (start 72.166 49.586) (end 72.166 37.126) (width 0.254) (layer "B.Cu") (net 2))
 (segment (start 72.166 37.126) (end 70.77 35.73) (width 0.254) (layer "B.Cu") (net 2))
 (segment (start 78.08 55.5) (end 72.166 49.586) (width 0.254) (layer "B.Cu") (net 2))
 (segment (start 76.34 81) (end 97 81) (width 0.254) (layer "F.Cu") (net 41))
 (segment (start 71.84 76.5) (end 76.34 81) (width 0.254) (layer "F.Cu") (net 41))
 (segment (start 97 81) (end 100 78) (width 0.254) (layer "F.Cu") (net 41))
 (segment (start 100 78) (end 100 62.08) (width 0.254) (layer "F.Cu") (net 41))
 (segment (start 100 62.08) (end 95.5 57.58) (width 0.254) (layer "F.Cu") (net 41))
 (segment (start 67 38.657861) (end 67 37.04) (width 0.254) (layer "F.Cu") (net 20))
 (segment (start 72.342139 44) (end 67 38.657861) (width 0.254) (layer "F.Cu") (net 20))
 (segment (start 67 37.04) (end 65.69 35.73) (width 0.254) (layer "F.Cu") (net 20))
 (segment (start 75.16 44) (end 72.342139 44) (width 0.254) (layer "F.Cu") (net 20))
 (segment (start 63.818 45.182) (end 65 44) (width 0.254) (layer "F.Cu") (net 4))
 (segment (start 51.182 45.182) (end 63.818 45.182) (width 0.254) (layer "F.Cu") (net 4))
 (segment (start 50 44) (end 51.182 45.182) (width 0.254) (layer "F.Cu") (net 4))
 (segment (start 59 50) (end 65 44) (width 0.254) (layer "B.Cu") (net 4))
 (segment (start 59 50.45) (end 59 50) (width 0.254) (layer "B.Cu") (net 4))
 (segment (start 78.39 35.73) (end 78.25 35.73) (width 0.254) (layer "B.Cu") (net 27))
 (segment (start 62.092768 49.068) (end 67.92 54.895232) (width 0.254) (layer "F.Cu") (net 1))
 (segment (start 67.92 54.895232) (end 67.92 55.5) (width 0.254) (layer "F.Cu") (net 1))
 (segment (start 53.92 56.5) (end 53.92 50.2735) (width 0.254) (layer "F.Cu") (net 1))
 (segment (start 53.92 50.2735) (end 55.1255 49.068) (width 0.254) (layer "F.Cu") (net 1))
 (segment (start 44.302 55.118) (end 52.538 55.118) (width 0.254) (layer "F.Cu") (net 1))
 (segment (start 55.1255 49.068) (end 62.092768 49.068) (width 0.254) (layer "F.Cu") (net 1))
 (segment (start 52.538 55.118) (end 53.92 56.5) (width 0.254) (layer "F.Cu") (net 1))
 (segment (start 42.92 56.5) (end 44.302 55.118) (width 0.254) (layer "F.Cu") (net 1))
 (segment (start 84.235 47.42) (end 82.695 48.96) (width 0.254) (layer "F.Cu") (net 37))
 (segment (start 95.5 47.42) (end 84.235 47.42) (width 0.254) (layer "F.Cu") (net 37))
 (segment (start 65.404 38.556) (end 65.69 38.27) (width 0.512) (layer "F.Cu") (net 19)))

